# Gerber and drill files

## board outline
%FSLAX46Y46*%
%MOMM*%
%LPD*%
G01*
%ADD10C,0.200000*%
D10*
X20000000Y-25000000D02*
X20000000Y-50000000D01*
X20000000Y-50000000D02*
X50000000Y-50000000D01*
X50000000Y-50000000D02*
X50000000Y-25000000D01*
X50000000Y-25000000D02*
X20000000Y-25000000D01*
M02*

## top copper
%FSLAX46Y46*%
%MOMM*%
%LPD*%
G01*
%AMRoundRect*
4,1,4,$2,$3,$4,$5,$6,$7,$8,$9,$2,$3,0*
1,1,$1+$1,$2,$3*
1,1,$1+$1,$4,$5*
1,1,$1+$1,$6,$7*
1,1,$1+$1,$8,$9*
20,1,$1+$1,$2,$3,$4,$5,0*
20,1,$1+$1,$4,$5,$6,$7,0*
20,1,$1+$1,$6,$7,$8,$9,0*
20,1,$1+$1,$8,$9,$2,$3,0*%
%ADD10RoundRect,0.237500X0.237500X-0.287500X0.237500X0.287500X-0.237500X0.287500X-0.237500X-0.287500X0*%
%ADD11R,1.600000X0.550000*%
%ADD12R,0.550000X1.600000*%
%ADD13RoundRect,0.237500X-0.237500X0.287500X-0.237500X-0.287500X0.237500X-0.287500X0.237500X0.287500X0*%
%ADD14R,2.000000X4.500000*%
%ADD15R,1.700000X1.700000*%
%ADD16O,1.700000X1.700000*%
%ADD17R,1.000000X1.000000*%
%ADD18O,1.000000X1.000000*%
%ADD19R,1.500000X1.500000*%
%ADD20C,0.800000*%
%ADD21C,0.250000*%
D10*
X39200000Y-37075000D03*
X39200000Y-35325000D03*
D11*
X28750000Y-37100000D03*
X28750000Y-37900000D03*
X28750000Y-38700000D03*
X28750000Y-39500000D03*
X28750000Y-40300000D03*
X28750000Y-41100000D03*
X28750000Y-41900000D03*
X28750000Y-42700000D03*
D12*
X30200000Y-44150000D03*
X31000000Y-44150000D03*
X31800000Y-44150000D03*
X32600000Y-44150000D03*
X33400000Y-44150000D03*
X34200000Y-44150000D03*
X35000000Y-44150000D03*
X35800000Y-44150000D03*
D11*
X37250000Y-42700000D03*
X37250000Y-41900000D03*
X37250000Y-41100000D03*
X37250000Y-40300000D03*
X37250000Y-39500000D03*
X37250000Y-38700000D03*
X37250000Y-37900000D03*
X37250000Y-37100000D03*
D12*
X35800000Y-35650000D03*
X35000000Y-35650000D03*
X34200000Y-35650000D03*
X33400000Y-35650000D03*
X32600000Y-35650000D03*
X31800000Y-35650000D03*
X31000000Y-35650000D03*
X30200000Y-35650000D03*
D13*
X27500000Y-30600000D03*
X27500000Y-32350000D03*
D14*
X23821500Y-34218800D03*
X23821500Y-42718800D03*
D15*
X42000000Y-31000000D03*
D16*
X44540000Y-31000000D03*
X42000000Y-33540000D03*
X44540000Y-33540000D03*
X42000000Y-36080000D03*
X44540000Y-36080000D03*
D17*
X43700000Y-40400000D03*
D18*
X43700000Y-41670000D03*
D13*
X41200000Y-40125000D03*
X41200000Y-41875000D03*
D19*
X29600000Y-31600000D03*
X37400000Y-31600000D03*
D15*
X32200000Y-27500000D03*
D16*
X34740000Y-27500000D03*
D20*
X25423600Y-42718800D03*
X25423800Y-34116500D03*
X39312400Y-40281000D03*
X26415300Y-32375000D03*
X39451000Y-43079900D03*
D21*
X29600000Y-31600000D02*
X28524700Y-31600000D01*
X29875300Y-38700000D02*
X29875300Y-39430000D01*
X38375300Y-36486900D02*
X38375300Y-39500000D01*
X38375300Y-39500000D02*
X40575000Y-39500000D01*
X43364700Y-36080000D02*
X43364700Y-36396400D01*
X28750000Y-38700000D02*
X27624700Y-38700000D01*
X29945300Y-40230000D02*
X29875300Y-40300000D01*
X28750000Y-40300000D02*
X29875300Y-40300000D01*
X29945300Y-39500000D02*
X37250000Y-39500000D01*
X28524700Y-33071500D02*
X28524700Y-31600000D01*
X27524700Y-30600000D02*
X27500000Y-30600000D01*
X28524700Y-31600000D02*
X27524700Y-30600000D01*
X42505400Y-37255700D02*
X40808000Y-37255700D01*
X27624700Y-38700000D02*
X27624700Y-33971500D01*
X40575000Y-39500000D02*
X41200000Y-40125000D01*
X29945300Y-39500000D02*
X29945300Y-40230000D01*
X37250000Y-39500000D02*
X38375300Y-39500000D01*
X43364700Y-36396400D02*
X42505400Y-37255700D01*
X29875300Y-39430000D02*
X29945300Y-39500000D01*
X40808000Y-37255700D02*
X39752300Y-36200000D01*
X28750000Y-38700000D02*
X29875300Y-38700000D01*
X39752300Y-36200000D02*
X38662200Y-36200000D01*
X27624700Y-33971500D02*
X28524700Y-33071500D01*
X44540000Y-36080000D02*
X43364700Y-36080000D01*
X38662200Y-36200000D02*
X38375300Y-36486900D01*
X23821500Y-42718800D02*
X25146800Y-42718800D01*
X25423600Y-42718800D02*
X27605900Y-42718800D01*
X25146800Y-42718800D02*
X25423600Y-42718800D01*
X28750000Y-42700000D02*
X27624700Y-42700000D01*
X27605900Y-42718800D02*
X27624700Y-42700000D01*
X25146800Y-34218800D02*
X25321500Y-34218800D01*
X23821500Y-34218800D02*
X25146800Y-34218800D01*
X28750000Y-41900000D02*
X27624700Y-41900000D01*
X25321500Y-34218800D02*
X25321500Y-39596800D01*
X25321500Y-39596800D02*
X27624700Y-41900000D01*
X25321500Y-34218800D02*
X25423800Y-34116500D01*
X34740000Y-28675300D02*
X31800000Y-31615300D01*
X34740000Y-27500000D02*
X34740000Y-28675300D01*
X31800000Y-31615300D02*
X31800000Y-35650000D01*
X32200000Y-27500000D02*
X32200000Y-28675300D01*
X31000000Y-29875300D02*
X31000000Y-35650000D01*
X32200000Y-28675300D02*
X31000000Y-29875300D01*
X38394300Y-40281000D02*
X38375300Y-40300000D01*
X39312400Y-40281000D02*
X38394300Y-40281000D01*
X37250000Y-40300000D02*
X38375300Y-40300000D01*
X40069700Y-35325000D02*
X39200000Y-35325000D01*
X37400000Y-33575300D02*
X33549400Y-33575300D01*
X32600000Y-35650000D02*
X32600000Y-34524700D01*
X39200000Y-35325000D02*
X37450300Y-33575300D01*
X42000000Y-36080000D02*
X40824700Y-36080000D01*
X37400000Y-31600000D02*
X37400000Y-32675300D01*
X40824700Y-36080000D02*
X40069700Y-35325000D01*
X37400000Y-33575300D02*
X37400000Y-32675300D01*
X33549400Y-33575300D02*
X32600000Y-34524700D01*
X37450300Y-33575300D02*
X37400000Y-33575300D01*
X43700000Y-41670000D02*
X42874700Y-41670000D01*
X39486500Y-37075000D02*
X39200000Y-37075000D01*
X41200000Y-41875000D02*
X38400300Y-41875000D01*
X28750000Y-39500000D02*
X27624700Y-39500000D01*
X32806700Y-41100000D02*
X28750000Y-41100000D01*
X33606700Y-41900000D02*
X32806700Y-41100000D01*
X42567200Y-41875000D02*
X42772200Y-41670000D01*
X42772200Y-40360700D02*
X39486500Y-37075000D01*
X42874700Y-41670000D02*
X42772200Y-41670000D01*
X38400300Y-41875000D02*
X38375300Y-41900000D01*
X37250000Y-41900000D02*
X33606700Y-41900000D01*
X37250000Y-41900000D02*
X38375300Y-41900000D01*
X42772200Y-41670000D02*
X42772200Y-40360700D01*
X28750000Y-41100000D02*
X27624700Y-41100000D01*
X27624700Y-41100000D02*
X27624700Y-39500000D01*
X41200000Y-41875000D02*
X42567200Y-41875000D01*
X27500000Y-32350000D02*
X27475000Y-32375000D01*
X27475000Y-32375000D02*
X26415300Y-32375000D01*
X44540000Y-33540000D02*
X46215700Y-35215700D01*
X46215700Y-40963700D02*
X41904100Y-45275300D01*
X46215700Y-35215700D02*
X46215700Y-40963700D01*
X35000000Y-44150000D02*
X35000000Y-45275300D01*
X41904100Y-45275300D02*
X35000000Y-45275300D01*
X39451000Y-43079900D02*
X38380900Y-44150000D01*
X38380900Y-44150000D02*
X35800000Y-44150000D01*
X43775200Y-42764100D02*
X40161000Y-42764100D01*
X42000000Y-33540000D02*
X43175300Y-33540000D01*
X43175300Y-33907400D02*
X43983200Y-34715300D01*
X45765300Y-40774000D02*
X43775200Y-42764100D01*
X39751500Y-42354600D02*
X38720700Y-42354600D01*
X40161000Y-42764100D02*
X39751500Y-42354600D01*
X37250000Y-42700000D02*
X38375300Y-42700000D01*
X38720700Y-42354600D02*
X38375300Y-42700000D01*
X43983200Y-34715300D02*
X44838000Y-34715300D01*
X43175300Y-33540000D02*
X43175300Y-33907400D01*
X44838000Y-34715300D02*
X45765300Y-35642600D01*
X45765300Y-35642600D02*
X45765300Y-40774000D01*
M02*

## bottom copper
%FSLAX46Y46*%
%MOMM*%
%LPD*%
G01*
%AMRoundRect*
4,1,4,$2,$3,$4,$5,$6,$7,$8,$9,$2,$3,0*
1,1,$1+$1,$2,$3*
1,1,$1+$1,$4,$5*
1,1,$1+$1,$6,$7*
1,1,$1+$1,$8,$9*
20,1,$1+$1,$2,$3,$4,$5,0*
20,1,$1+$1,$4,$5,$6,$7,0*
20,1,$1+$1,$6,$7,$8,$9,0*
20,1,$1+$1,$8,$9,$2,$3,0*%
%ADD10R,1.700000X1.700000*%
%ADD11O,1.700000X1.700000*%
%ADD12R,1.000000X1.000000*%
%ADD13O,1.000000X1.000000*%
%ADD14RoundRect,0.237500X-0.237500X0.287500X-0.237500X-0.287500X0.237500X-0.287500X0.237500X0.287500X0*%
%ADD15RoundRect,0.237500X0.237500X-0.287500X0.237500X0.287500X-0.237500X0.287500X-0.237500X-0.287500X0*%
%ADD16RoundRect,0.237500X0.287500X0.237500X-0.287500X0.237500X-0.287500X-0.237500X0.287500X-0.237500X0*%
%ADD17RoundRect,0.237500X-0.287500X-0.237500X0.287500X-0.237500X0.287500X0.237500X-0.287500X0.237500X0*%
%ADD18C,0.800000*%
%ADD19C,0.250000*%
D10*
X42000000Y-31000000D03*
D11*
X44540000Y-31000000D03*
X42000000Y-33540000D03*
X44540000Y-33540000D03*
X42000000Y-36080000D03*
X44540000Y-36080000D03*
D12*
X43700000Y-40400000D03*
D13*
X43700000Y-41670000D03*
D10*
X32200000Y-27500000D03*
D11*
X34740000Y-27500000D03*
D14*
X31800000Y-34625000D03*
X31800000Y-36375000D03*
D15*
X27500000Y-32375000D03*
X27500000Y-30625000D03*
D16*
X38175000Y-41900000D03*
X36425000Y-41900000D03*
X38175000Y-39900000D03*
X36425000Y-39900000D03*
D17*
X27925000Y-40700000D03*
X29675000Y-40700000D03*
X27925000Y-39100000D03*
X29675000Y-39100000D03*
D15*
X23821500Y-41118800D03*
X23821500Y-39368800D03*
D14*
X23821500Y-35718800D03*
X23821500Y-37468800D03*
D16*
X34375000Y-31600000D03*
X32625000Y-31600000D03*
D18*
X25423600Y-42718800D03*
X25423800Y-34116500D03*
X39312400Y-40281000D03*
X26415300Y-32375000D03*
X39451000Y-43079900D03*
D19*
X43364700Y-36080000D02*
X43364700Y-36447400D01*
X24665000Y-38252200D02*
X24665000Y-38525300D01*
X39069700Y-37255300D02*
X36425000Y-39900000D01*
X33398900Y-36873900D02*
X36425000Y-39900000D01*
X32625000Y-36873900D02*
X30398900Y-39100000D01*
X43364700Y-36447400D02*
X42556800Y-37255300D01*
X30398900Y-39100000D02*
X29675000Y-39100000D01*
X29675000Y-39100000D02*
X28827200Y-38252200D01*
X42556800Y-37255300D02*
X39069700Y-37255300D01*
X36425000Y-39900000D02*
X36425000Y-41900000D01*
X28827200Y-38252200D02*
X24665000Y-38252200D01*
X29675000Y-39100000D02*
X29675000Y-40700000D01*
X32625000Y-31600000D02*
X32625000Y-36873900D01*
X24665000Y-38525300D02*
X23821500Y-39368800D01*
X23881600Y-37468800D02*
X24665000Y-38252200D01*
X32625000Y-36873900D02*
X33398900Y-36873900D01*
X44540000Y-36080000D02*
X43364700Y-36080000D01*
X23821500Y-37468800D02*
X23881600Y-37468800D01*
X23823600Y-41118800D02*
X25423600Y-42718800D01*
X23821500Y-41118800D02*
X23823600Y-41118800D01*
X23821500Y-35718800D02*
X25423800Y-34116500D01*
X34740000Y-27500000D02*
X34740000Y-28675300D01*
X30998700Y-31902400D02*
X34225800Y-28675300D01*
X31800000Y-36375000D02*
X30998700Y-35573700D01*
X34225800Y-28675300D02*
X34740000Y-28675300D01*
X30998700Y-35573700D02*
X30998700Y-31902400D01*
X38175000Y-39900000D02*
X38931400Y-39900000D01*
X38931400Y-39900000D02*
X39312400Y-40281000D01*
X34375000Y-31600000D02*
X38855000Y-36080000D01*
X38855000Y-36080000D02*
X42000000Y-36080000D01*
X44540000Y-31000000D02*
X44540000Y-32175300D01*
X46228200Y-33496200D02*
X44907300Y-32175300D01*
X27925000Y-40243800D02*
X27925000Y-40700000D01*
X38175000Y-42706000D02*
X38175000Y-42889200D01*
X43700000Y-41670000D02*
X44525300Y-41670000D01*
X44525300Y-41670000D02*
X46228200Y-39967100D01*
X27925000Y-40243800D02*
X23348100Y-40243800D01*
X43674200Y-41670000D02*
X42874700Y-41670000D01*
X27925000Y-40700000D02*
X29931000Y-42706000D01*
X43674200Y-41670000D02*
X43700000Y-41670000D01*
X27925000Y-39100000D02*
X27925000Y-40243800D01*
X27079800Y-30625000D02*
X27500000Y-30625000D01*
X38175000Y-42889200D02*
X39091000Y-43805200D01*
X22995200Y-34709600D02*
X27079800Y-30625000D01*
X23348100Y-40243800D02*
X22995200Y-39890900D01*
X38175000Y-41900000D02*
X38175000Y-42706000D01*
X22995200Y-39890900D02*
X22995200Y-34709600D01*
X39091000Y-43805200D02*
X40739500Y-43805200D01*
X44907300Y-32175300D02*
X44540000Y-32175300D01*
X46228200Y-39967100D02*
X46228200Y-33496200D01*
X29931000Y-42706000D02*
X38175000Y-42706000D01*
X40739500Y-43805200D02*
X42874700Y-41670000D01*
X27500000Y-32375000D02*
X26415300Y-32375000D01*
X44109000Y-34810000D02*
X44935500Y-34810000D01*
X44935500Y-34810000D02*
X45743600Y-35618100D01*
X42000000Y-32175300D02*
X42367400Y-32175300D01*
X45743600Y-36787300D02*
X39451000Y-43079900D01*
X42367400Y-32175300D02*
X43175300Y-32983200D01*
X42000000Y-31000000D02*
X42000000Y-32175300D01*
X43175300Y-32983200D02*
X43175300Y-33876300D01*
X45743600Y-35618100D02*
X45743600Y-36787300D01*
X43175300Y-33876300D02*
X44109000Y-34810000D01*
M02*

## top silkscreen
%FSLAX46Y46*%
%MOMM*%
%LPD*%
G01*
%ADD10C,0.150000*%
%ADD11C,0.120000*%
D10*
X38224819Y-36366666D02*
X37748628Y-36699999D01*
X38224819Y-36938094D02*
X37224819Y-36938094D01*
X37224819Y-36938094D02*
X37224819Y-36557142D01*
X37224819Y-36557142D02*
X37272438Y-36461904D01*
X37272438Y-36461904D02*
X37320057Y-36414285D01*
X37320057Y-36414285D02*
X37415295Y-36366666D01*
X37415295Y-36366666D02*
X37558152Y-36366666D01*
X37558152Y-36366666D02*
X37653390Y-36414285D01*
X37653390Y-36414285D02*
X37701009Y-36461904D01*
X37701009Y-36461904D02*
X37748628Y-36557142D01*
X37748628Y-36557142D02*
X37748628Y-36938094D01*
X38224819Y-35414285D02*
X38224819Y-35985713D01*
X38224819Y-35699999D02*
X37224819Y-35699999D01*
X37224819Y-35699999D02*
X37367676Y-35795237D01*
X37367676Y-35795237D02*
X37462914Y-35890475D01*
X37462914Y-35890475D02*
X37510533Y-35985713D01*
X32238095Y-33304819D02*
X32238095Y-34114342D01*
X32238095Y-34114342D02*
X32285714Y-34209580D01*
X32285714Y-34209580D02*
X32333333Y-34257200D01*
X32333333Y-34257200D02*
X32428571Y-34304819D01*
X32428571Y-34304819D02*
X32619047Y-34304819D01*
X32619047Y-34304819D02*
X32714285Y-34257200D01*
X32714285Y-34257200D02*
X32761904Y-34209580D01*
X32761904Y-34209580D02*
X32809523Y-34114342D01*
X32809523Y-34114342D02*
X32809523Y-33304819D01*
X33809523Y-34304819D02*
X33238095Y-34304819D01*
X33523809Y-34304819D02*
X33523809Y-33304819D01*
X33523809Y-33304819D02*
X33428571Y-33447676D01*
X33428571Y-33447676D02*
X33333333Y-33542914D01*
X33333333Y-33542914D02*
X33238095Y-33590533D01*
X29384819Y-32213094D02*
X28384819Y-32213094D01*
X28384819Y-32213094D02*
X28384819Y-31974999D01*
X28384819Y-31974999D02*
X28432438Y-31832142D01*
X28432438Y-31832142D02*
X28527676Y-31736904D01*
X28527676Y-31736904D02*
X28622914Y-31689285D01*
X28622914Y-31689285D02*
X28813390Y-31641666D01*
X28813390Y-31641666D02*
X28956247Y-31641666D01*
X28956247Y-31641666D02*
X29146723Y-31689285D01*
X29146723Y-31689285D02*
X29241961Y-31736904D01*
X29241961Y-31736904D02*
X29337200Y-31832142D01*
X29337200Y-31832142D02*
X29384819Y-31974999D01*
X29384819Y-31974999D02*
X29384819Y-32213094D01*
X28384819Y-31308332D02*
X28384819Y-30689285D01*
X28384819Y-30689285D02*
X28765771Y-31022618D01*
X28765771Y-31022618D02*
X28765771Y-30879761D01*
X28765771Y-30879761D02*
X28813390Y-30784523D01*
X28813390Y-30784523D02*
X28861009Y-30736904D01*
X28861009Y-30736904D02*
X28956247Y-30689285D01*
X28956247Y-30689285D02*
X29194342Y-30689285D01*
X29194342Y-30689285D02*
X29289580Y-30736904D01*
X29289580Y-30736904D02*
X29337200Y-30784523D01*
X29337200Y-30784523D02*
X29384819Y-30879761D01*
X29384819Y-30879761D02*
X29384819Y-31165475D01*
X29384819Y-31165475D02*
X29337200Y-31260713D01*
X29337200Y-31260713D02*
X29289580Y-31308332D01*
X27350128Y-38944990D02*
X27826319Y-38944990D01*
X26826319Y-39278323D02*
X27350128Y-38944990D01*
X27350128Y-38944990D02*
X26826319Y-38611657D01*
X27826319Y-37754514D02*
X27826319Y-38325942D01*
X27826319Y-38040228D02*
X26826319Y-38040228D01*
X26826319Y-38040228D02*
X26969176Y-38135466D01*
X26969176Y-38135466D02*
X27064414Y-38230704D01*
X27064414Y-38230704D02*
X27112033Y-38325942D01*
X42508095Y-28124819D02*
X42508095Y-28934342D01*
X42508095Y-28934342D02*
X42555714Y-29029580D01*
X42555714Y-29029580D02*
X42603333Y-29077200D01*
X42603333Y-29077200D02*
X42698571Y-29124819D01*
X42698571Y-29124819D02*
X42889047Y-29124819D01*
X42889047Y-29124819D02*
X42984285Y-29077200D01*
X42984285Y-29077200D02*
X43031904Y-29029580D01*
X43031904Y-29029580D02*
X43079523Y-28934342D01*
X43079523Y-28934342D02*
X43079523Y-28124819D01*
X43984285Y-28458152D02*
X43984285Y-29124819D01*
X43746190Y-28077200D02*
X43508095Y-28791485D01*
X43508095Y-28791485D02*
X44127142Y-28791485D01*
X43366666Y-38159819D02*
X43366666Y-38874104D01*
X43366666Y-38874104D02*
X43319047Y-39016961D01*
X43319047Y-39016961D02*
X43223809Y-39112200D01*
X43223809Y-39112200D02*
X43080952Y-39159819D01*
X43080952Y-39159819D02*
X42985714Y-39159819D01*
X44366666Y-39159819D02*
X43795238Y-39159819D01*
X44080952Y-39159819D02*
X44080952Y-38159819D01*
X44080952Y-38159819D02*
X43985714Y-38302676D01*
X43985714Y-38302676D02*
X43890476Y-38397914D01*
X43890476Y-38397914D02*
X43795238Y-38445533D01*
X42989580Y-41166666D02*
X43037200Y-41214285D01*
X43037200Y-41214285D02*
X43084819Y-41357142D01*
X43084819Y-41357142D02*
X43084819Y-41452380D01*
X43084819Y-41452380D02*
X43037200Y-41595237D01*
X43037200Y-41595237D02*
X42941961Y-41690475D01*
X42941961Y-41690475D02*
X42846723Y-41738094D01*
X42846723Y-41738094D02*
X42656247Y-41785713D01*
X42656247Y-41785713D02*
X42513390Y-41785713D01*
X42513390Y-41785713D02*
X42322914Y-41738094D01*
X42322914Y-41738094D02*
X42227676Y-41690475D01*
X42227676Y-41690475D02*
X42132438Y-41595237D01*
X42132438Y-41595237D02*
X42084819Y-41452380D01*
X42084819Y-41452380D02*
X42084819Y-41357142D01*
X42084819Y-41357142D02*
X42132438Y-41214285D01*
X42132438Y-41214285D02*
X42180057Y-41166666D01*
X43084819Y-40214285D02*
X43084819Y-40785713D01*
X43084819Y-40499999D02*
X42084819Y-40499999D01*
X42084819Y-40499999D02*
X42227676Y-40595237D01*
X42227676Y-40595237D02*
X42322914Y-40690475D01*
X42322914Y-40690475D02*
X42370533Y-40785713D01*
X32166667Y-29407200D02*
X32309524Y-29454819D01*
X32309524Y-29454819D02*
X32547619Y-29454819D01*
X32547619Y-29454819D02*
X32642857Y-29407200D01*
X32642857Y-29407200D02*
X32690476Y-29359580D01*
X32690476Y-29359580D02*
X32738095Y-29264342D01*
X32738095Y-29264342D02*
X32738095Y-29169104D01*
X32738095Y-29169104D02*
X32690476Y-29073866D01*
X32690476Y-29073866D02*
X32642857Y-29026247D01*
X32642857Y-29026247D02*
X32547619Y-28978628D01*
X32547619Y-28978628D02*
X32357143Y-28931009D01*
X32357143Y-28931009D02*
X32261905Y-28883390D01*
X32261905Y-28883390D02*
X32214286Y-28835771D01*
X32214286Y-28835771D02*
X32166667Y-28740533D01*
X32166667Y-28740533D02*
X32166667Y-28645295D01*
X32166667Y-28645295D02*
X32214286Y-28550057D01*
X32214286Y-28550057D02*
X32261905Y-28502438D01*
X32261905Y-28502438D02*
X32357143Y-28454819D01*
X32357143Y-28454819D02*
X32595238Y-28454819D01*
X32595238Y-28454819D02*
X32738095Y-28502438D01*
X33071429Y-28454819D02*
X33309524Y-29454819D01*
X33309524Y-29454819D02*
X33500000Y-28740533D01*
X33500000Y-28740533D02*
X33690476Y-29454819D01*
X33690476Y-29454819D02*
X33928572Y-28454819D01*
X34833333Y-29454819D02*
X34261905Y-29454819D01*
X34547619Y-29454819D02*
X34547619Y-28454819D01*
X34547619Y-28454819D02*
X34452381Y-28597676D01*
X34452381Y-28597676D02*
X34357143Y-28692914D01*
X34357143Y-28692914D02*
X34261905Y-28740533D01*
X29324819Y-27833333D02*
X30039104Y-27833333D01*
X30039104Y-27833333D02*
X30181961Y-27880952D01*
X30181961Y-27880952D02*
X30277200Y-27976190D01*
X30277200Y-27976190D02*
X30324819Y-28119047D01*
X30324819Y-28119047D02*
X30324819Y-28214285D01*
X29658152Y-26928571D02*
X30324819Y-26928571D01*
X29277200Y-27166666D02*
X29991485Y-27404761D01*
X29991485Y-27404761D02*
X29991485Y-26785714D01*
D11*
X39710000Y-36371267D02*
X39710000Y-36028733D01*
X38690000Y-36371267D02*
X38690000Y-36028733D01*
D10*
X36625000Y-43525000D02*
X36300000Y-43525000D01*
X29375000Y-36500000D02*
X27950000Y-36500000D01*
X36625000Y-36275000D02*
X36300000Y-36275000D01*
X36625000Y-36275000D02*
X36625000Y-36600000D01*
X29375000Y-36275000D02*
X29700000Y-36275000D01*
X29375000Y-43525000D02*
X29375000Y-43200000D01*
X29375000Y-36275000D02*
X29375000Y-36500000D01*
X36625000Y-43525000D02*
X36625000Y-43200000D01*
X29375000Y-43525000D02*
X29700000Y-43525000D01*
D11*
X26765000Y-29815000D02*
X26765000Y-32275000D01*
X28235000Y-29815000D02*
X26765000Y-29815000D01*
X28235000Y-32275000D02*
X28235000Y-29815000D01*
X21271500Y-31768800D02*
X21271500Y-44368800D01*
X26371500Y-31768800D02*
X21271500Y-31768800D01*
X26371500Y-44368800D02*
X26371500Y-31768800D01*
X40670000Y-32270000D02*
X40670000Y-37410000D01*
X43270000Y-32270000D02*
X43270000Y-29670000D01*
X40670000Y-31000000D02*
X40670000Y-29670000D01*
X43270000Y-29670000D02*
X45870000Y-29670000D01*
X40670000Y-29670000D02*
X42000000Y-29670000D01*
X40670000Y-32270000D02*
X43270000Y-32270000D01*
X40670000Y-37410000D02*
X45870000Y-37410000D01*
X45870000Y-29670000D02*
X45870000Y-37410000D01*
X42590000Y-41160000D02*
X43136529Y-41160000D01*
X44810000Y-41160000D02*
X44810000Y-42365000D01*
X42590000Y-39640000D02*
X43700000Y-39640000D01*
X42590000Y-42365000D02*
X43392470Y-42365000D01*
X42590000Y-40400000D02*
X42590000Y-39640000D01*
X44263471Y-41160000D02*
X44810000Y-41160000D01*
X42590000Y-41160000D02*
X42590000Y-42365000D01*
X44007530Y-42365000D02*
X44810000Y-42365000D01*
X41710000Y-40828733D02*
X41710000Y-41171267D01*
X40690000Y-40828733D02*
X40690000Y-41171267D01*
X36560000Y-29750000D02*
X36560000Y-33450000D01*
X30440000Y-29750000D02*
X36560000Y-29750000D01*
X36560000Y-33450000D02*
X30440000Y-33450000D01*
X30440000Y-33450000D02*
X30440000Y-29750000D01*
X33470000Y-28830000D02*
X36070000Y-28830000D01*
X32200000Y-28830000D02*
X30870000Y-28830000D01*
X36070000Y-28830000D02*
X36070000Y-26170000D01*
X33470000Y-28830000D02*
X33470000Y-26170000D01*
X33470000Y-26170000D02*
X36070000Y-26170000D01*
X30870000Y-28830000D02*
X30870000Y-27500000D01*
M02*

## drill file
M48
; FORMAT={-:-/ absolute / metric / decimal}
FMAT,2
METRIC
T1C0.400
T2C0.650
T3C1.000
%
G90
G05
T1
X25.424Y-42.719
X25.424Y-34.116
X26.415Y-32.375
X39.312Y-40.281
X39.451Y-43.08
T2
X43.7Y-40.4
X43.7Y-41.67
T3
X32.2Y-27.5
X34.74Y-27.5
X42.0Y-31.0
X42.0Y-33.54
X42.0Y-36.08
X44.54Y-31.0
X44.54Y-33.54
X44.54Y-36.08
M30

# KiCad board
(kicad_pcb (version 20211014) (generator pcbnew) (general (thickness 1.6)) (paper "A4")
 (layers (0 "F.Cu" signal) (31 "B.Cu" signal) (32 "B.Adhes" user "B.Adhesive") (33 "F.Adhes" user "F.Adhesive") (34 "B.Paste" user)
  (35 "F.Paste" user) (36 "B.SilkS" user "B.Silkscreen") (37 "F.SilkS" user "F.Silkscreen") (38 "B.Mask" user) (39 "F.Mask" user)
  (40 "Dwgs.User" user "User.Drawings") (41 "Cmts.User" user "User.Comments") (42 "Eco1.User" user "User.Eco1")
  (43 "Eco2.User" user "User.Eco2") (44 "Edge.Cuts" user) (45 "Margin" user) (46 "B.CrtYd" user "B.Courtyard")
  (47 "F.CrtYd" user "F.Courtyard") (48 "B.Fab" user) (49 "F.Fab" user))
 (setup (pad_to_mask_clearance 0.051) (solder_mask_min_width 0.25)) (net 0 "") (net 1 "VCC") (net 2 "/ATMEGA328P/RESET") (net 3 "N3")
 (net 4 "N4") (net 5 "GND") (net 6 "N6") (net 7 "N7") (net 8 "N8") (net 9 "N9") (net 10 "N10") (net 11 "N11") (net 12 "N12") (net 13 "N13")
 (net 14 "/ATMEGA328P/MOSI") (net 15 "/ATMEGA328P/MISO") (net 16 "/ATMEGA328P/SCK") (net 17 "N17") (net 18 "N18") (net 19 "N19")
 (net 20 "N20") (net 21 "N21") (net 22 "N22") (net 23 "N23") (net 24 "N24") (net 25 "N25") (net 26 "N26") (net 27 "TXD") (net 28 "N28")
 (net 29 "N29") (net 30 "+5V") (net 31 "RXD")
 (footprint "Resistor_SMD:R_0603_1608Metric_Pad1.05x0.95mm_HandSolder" (layer "F.Cu") (at 39.2 36.2 90)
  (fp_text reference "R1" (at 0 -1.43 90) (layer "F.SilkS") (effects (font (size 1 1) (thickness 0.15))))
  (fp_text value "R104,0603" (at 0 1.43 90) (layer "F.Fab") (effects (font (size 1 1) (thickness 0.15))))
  (fp_line (start -0.171267 0.51) (end 0.171267 0.51) (layer "F.SilkS") (width 0.12))
  (fp_line (start -0.171267 -0.51) (end 0.171267 -0.51) (layer "F.SilkS") (width 0.12))
  (pad "1" smd roundrect locked (at -0.875 0 90) (size 1.05 0.95) (layers "F.Cu" "F.Paste" "F.Mask") (roundrect_rratio 0.25) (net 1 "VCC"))
  (pad "2" smd roundrect locked (at 0.875 0 90) (size 1.05 0.95) (layers "F.Cu" "F.Paste" "F.Mask") (roundrect_rratio 0.25)
   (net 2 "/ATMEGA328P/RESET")))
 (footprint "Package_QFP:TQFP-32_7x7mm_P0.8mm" (layer "F.Cu") (at 33 39.9)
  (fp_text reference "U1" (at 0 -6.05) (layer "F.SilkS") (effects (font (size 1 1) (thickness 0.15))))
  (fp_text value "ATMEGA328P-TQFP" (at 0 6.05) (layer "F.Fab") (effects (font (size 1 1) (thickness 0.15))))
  (fp_line (start 3.625 3.625) (end 3.3 3.625) (layer "F.SilkS") (width 0.15))
  (fp_line (start -3.625 -3.4) (end -5.05 -3.4) (layer "F.SilkS") (width 0.15))
  (fp_line (start 3.625 -3.625) (end 3.3 -3.625) (layer "F.SilkS") (width 0.15))
  (fp_line (start 3.625 -3.625) (end 3.625 -3.3) (layer "F.SilkS") (width 0.15))
  (fp_line (start -3.625 -3.625) (end -3.3 -3.625) (layer "F.SilkS") (width 0.15))
  (fp_line (start -3.625 3.625) (end -3.625 3.3) (layer "F.SilkS") (width 0.15))
  (fp_line (start -3.625 -3.625) (end -3.625 -3.4) (layer "F.SilkS") (width 0.15))
  (fp_line (start 3.625 3.625) (end 3.625 3.3) (layer "F.SilkS") (width 0.15))
  (fp_line (start -3.625 3.625) (end -3.3 3.625) (layer "F.SilkS") (width 0.15))
  (pad "1" smd rect locked (at -4.25 -2.8) (size 1.6 0.55) (layers "F.Cu" "F.Paste" "F.Mask") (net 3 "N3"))
  (pad "2" smd rect locked (at -4.25 -2) (size 1.6 0.55) (layers "F.Cu" "F.Paste" "F.Mask") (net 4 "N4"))
  (pad "3" smd rect locked (at -4.25 -1.2) (size 1.6 0.55) (layers "F.Cu" "F.Paste" "F.Mask") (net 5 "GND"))
  (pad "4" smd rect locked (at -4.25 -0.4) (size 1.6 0.55) (layers "F.Cu" "F.Paste" "F.Mask") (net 1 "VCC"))
  (pad "5" smd rect locked (at -4.25 0.4) (size 1.6 0.55) (layers "F.Cu" "F.Paste" "F.Mask") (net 5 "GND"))
  (pad "6" smd rect locked (at -4.25 1.2) (size 1.6 0.55) (layers "F.Cu" "F.Paste" "F.Mask") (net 1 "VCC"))
  (pad "7" smd rect locked (at -4.25 2) (size 1.6 0.55) (layers "F.Cu" "F.Paste" "F.Mask") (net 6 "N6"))
  (pad "8" smd rect locked (at -4.25 2.8) (size 1.6 0.55) (layers "F.Cu" "F.Paste" "F.Mask") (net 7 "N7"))
  (pad "9" smd rect locked (at -2.8 4.25 90) (size 1.6 0.55) (layers "F.Cu" "F.Paste" "F.Mask") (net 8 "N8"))
  (pad "10" smd rect locked (at -2 4.25 90) (size 1.6 0.55) (layers "F.Cu" "F.Paste" "F.Mask") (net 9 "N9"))
  (pad "11" smd rect locked (at -1.2 4.25 90) (size 1.6 0.55) (layers "F.Cu" "F.Paste" "F.Mask") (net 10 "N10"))
  (pad "12" smd rect locked (at -0.4 4.25 90) (size 1.6 0.55) (layers "F.Cu" "F.Paste" "F.Mask") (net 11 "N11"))
  (pad "13" smd rect locked (at 0.4 4.25 90) (size 1.6 0.55) (layers "F.Cu" "F.Paste" "F.Mask") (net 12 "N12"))
  (pad "14" smd rect locked (at 1.2 4.25 90) (size 1.6 0.55) (layers "F.Cu" "F.Paste" "F.Mask") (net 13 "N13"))
  (pad "15" smd rect locked (at 2 4.25 90) (size 1.6 0.55) (layers "F.Cu" "F.Paste" "F.Mask") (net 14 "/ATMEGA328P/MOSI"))
  (pad "16" smd rect locked (at 2.8 4.25 90) (size 1.6 0.55) (layers "F.Cu" "F.Paste" "F.Mask") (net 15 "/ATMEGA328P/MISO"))
  (pad "17" smd rect locked (at 4.25 2.8) (size 1.6 0.55) (layers "F.Cu" "F.Paste" "F.Mask") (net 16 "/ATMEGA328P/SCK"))
  (pad "18" smd rect locked (at 4.25 2) (size 1.6 0.55) (layers "F.Cu" "F.Paste" "F.Mask") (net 1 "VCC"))
  (pad "19" smd rect locked (at 4.25 1.2) (size 1.6 0.55) (layers "F.Cu" "F.Paste" "F.Mask") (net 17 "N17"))
  (pad "20" smd rect locked (at 4.25 0.4) (size 1.6 0.55) (layers "F.Cu" "F.Paste" "F.Mask") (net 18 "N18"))
  (pad "21" smd rect locked (at 4.25 -0.4) (size 1.6 0.55) (layers "F.Cu" "F.Paste" "F.Mask") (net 5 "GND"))
  (pad "22" smd rect locked (at 4.25 -1.2) (size 1.6 0.55) (layers "F.Cu" "F.Paste" "F.Mask") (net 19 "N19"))
  (pad "23" smd rect locked (at 4.25 -2) (size 1.6 0.55) (layers "F.Cu" "F.Paste" "F.Mask") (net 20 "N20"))
  (pad "24" smd rect locked (at 4.25 -2.8) (size 1.6 0.55) (layers "F.Cu" "F.Paste" "F.Mask") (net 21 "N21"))
  (pad "25" smd rect locked (at 2.8 -4.25 90) (size 1.6 0.55) (layers "F.Cu" "F.Paste" "F.Mask") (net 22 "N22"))
  (pad "26" smd rect locked (at 2 -4.25 90) (size 1.6 0.55) (layers "F.Cu" "F.Paste" "F.Mask") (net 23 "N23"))
  (pad "27" smd rect locked (at 1.2 -4.25 90) (size 1.6 0.55) (layers "F.Cu" "F.Paste" "F.Mask") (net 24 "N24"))
  (pad "28" smd rect locked (at 0.4 -4.25 90) (size 1.6 0.55) (layers "F.Cu" "F.Paste" "F.Mask") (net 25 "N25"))
  (pad "29" smd rect locked (at -0.4 -4.25 90) (size 1.6 0.55) (layers "F.Cu" "F.Paste" "F.Mask") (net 2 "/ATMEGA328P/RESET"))
  (pad "30" smd rect locked (at -1.2 -4.25 90) (size 1.6 0.55) (layers "F.Cu" "F.Paste" "F.Mask") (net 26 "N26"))
  (pad "31" smd rect locked (at -2 -4.25 90) (size 1.6 0.55) (layers "F.Cu" "F.Paste" "F.Mask") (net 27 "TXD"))
  (pad "32" smd rect locked (at -2.8 -4.25 90) (size 1.6 0.55) (layers "F.Cu" "F.Paste" "F.Mask") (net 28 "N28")))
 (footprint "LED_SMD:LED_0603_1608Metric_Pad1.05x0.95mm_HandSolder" (layer "F.Cu") (at 27.5 31.475 -90)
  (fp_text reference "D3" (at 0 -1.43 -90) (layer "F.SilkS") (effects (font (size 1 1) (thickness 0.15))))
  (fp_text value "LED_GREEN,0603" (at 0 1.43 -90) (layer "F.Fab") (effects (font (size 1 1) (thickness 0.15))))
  (fp_line (start -1.66 0.735) (end 0.8 0.735) (layer "F.SilkS") (width 0.12))
  (fp_line (start -1.66 -0.735) (end -1.66 0.735) (layer "F.SilkS") (width 0.12))
  (fp_line (start 0.8 -0.735) (end -1.66 -0.735) (layer "F.SilkS") (width 0.12))
  (pad "1" smd roundrect locked (at -0.875 0 270) (size 1.05 0.95) (layers "F.Cu" "F.Paste" "F.Mask") (roundrect_rratio 0.25) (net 5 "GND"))
  (pad "2" smd roundrect locked (at 0.875 0 270) (size 1.05 0.95) (layers "F.Cu" "F.Paste" "F.Mask") (roundrect_rratio 0.25) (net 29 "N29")))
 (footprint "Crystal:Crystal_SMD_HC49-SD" (layer "F.Cu") (at 23.8215 38.4688 -90)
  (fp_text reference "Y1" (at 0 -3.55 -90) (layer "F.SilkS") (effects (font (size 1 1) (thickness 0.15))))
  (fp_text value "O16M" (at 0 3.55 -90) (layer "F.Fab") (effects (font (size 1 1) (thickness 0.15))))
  (fp_line (start -6.7 2.55) (end 5.9 2.55) (layer "F.SilkS") (width 0.12))
  (fp_line (start -6.7 -2.55) (end -6.7 2.55) (layer "F.SilkS") (width 0.12))
  (fp_line (start 5.9 -2.55) (end -6.7 -2.55) (layer "F.SilkS") (width 0.12))
  (pad "1" smd rect locked (at -4.25 0 270) (size 4.5 2) (layers "F.Cu" "F.Paste" "F.Mask") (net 6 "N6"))
  (pad "2" smd rect locked (at 4.25 0 270) (size 4.5 2) (layers "F.Cu" "F.Paste" "F.Mask") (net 7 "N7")))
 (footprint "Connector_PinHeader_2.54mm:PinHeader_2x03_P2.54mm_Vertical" (layer "F.Cu") (at 42 31)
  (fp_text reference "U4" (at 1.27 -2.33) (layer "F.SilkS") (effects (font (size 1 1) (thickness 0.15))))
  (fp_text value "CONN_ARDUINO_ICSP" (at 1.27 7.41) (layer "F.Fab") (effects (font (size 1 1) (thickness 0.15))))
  (fp_line (start -1.33 1.27) (end -1.33 6.41) (layer "F.SilkS") (width 0.12))
  (fp_line (start 1.27 1.27) (end 1.27 -1.33) (layer "F.SilkS") (width 0.12))
  (fp_line (start -1.33 0) (end -1.33 -1.33) (layer "F.SilkS") (width 0.12))
  (fp_line (start 1.27 -1.33) (end 3.87 -1.33) (layer "F.SilkS") (width 0.12))
  (fp_line (start -1.33 -1.33) (end 0 -1.33) (layer "F.SilkS") (width 0.12))
  (fp_line (start -1.33 1.27) (end 1.27 1.27) (layer "F.SilkS") (width 0.12))
  (fp_line (start -1.33 6.41) (end 3.87 6.41) (layer "F.SilkS") (width 0.12))
  (fp_line (start 3.87 -1.33) (end 3.87 6.41) (layer "F.SilkS") (width 0.12))
  (pad "1" thru_hole rect locked (at 0 0) (size 1.7 1.7) (drill 1) (layers *.Cu *.Mask) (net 15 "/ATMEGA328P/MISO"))
  (pad "2" thru_hole oval locked (at 2.54 0) (size 1.7 1.7) (drill 1) (layers *.Cu *.Mask) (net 1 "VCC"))
  (pad "3" thru_hole oval locked (at 0 2.54) (size 1.7 1.7) (drill 1) (layers *.Cu *.Mask) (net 16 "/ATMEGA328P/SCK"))
  (pad "4" thru_hole oval locked (at 2.54 2.54) (size 1.7 1.7) (drill 1) (layers *.Cu *.Mask) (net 14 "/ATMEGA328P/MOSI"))
  (pad "5" thru_hole oval locked (at 0 5.08) (size 1.7 1.7) (drill 1) (layers *.Cu *.Mask) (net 2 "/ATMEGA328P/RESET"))
  (pad "6" thru_hole oval locked (at 2.54 5.08) (size 1.7 1.7) (drill 1) (layers *.Cu *.Mask) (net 5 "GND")))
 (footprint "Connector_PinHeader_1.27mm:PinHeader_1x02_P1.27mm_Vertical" (layer "F.Cu") (at 43.7 40.4)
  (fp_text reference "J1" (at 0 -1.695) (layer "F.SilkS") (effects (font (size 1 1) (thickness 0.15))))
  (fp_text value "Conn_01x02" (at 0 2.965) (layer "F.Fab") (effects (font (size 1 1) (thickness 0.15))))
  (fp_line (start -1.11 0.76) (end -0.563471 0.76) (layer "F.SilkS") (width 0.12))
  (fp_line (start 1.11 0.76) (end 1.11 1.965) (layer "F.SilkS") (width 0.12))
  (fp_line (start -1.11 -0.76) (end 0 -0.76) (layer "F.SilkS") (width 0.12))
  (fp_line (start -1.11 1.965) (end -0.30753 1.965) (layer "F.SilkS") (width 0.12))
  (fp_line (start -1.11 0) (end -1.11 -0.76) (layer "F.SilkS") (width 0.12))
  (fp_line (start 0.563471 0.76) (end 1.11 0.76) (layer "F.SilkS") (width 0.12))
  (fp_line (start -1.11 0.76) (end -1.11 1.965) (layer "F.SilkS") (width 0.12))
  (fp_line (start 0.30753 1.965) (end 1.11 1.965) (layer "F.SilkS") (width 0.12))
  (pad "1" thru_hole rect locked (at 0 0) (size 1 1) (drill 0.65) (layers *.Cu *.Mask) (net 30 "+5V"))
  (pad "2" thru_hole oval locked (at 0 1.27) (size 1 1) (drill 0.65) (layers *.Cu *.Mask) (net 1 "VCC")))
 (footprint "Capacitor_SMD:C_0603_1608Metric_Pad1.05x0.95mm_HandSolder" (layer "F.Cu") (at 41.2 41 -90)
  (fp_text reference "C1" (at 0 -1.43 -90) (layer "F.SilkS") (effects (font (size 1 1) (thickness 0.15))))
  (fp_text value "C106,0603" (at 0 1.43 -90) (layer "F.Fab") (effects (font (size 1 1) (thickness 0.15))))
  (fp_line (start -0.171267 -0.51) (end 0.171267 -0.51) (layer "F.SilkS") (width 0.12))
  (fp_line (start -0.171267 0.51) (end 0.171267 0.51) (layer "F.SilkS") (width 0.12))
  (pad "1" smd roundrect locked (at -0.875 0 270) (size 1.05 0.95) (layers "F.Cu" "F.Paste" "F.Mask") (roundrect_rratio 0.25) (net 5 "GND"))
  (pad "2" smd roundrect locked (at 0.875 0 270) (size 1.05 0.95) (layers "F.Cu" "F.Paste" "F.Mask") (roundrect_rratio 0.25) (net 1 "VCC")))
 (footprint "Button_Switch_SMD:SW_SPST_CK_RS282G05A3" (layer "F.Cu") (at 33.5 31.6)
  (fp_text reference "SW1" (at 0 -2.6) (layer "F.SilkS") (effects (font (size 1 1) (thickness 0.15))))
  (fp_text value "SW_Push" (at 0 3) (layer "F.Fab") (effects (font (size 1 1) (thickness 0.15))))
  (fp_line (start 3.06 -1.85) (end 3.06 1.85) (layer "F.SilkS") (width 0.12))
  (fp_line (start -3.06 -1.85) (end 3.06 -1.85) (layer "F.SilkS") (width 0.12))
  (fp_line (start 3.06 1.85) (end -3.06 1.85) (layer "F.SilkS") (width 0.12))
  (fp_line (start -3.06 1.85) (end -3.06 -1.85) (layer "F.SilkS") (width 0.12))
  (pad "1" smd rect locked (at -3.9 0) (size 1.5 1.5) (layers "F.Cu" "F.Paste" "F.Mask") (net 5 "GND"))
  (pad "2" smd rect locked (at 3.9 0) (size 1.5 1.5) (layers "F.Cu" "F.Paste" "F.Mask") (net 2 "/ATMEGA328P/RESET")))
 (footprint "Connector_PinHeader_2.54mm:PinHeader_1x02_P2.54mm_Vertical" (layer "F.Cu") (at 32.2 27.5 90)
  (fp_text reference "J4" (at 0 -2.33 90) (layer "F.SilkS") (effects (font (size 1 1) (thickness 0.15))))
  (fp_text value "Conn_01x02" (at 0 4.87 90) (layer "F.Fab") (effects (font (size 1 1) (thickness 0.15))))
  (fp_line (start -1.33 1.27) (end -1.33 3.87) (layer "F.SilkS") (width 0.12))
  (fp_line (start -1.33 0) (end -1.33 -1.33) (layer "F.SilkS") (width 0.12))
  (fp_line (start -1.33 3.87) (end 1.33 3.87) (layer "F.SilkS") (width 0.12))
  (fp_line (start -1.33 1.27) (end 1.33 1.27) (layer "F.SilkS") (width 0.12))
  (fp_line (start 1.33 1.27) (end 1.33 3.87) (layer "F.SilkS") (width 0.12))
  (fp_line (start -1.33 -1.33) (end 0 -1.33) (layer "F.SilkS") (width 0.12))
  (pad "1" thru_hole rect locked (at 0 0 90) (size 1.7 1.7) (drill 1) (layers *.Cu *.Mask) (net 27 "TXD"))
  (pad "2" thru_hole oval locked (at 0 2.54 90) (size 1.7 1.7) (drill 1) (layers *.Cu *.Mask) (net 26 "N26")))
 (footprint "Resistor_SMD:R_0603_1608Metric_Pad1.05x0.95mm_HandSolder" (layer "B.Cu") (at 31.8 35.5 -90)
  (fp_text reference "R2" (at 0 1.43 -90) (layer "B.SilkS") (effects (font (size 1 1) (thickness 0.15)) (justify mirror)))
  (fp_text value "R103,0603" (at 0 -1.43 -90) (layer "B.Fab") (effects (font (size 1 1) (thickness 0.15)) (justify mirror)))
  (pad "1" smd roundrect locked (at -0.875 0 270) (size 1.05 0.95) (layers "B.Cu" "B.Paste" "B.Mask") (roundrect_rratio 0.25) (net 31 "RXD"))
  (pad "2" smd roundrect locked (at 0.875 0 270) (size 1.05 0.95) (layers "B.Cu" "B.Paste" "B.Mask") (roundrect_rratio 0.25) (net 26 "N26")))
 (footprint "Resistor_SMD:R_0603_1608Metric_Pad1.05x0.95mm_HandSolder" (layer "B.Cu") (at 27.5 31.5 90)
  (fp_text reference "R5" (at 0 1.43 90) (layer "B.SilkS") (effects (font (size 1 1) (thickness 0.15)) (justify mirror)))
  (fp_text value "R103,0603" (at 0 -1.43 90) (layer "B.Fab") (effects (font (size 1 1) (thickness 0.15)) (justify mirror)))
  (pad "1" smd roundrect locked (at -0.875 0 90) (size 1.05 0.95) (layers "B.Cu" "B.Paste" "B.Mask") (roundrect_rratio 0.25) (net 29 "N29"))
  (pad "2" smd roundrect locked (at 0.875 0 90) (size 1.05 0.95) (layers "B.Cu" "B.Paste" "B.Mask") (roundrect_rratio 0.25) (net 1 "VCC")))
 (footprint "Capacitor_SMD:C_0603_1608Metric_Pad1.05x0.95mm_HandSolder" (layer "B.Cu") (at 37.3 41.9 180)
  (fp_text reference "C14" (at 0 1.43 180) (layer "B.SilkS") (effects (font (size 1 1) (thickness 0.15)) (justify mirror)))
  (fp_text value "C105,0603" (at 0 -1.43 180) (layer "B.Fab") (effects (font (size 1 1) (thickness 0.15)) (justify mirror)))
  (pad "1" smd roundrect locked (at -0.875 0 180) (size 1.05 0.95) (layers "B.Cu" "B.Paste" "B.Mask") (roundrect_rratio 0.25) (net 1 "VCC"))
  (pad "2" smd roundrect locked (at 0.875 0 180) (size 1.05 0.95) (layers "B.Cu" "B.Paste" "B.Mask") (roundrect_rratio 0.25) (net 5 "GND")))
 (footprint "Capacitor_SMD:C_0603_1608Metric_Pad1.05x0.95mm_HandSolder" (layer "B.Cu") (at 37.3 39.9 180)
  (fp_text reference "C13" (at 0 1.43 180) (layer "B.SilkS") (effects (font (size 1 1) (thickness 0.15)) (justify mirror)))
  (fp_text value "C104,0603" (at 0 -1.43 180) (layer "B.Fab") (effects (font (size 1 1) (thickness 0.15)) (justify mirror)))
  (pad "1" smd roundrect locked (at -0.875 0 180) (size 1.05 0.95) (layers "B.Cu" "B.Paste" "B.Mask") (roundrect_rratio 0.25) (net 18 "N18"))
  (pad "2" smd roundrect locked (at 0.875 0 180) (size 1.05 0.95) (layers "B.Cu" "B.Paste" "B.Mask") (roundrect_rratio 0.25) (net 5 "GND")))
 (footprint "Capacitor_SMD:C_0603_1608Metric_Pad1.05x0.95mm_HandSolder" (layer "B.Cu") (at 28.8 40.7)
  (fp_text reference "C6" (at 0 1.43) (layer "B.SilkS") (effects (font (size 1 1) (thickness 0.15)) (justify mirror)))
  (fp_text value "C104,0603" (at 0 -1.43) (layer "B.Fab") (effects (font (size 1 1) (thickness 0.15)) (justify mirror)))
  (pad "1" smd roundrect locked (at -0.875 0) (size 1.05 0.95) (layers "B.Cu" "B.Paste" "B.Mask") (roundrect_rratio 0.25) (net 1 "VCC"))
  (pad "2" smd roundrect locked (at 0.875 0) (size 1.05 0.95) (layers "B.Cu" "B.Paste" "B.Mask") (roundrect_rratio 0.25) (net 5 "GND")))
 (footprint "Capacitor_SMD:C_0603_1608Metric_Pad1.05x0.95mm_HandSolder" (layer "B.Cu") (at 28.8 39.1)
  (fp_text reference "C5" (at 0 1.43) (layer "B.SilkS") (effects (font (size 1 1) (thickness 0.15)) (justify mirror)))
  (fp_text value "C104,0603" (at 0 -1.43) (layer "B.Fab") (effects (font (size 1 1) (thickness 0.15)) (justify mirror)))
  (pad "1" smd roundrect locked (at -0.875 0) (size 1.05 0.95) (layers "B.Cu" "B.Paste" "B.Mask") (roundrect_rratio 0.25) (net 1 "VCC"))
  (pad "2" smd roundrect locked (at 0.875 0) (size 1.05 0.95) (layers "B.Cu" "B.Paste" "B.Mask") (roundrect_rratio 0.25) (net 5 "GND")))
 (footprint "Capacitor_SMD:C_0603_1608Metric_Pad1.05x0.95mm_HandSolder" (layer "B.Cu") (at 23.8215 40.2438 90)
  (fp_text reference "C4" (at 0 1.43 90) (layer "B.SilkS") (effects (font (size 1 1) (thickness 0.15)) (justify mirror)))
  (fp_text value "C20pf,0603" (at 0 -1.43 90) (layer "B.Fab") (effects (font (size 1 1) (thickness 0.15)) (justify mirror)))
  (pad "1" smd roundrect locked (at -0.875 0 90) (size 1.05 0.95) (layers "B.Cu" "B.Paste" "B.Mask") (roundrect_rratio 0.25) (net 7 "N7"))
  (pad "2" smd roundrect locked (at 0.875 0 90) (size 1.05 0.95) (layers "B.Cu" "B.Paste" "B.Mask") (roundrect_rratio 0.25) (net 5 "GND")))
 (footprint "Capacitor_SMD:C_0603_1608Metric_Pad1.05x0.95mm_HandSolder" (layer "B.Cu") (at 23.8215 36.5938 -90)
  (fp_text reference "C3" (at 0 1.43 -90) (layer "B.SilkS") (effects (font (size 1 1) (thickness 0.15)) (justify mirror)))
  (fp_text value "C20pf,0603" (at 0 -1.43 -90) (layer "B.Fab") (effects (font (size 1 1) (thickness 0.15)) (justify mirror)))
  (pad "1" smd roundrect locked (at -0.875 0 270) (size 1.05 0.95) (layers "B.Cu" "B.Paste" "B.Mask") (roundrect_rratio 0.25) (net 6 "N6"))
  (pad "2" smd roundrect locked (at 0.875 0 270) (size 1.05 0.95) (layers "B.Cu" "B.Paste" "B.Mask") (roundrect_rratio 0.25) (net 5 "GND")))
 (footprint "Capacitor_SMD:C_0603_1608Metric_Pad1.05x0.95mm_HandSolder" (layer "B.Cu") (at 33.5 31.6 180)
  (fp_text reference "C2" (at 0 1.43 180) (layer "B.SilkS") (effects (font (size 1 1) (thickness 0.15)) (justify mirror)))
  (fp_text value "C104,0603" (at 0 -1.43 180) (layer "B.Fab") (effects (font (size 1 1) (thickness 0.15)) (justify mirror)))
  (pad "1" smd roundrect locked (at -0.875 0 180) (size 1.05 0.95) (layers "B.Cu" "B.Paste" "B.Mask") (roundrect_rratio 0.25)
   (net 2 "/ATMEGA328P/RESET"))
  (pad "2" smd roundrect locked (at 0.875 0 180) (size 1.05 0.95) (layers "B.Cu" "B.Paste" "B.Mask") (roundrect_rratio 0.25) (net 5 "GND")))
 (gr_line (start 20 25) (end 20 50) (layer "Edge.Cuts") (width 0.2))
 (gr_line (start 20 50) (end 50 50) (layer "Edge.Cuts") (width 0.2))
 (gr_line (start 50 50) (end 50 25) (layer "Edge.Cuts") (width 0.2))
 (gr_line (start 50 25) (end 20 25) (layer "Edge.Cuts") (width 0.2))
 (segment (start 29.6 31.6) (end 28.5247 31.6) (width 0.25) (layer "F.Cu") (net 5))
 (segment (start 29.8753 38.7) (end 29.8753 39.43) (width 0.25) (layer "F.Cu") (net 5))
 (segment (start 38.3753 36.4869) (end 38.3753 39.5) (width 0.25) (layer "F.Cu") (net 5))
 (segment (start 38.3753 39.5) (end 40.575 39.5) (width 0.25) (layer "F.Cu") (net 5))
 (segment (start 43.3647 36.08) (end 43.3647 36.3964) (width 0.25) (layer "F.Cu") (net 5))
 (segment (start 28.75 38.7) (end 27.6247 38.7) (width 0.25) (layer "F.Cu") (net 5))
 (segment (start 29.9453 40.23) (end 29.8753 40.3) (width 0.25) (layer "F.Cu") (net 5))
 (segment (start 28.75 40.3) (end 29.8753 40.3) (width 0.25) (layer "F.Cu") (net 5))
 (segment (start 29.9453 39.5) (end 37.25 39.5) (width 0.25) (layer "F.Cu") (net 5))
 (segment (start 28.5247 33.0715) (end 28.5247 31.6) (width 0.25) (layer "F.Cu") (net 5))
 (segment (start 27.5247 30.6) (end 27.5 30.6) (width 0.25) (layer "F.Cu") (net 5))
 (segment (start 28.5247 31.6) (end 27.5247 30.6) (width 0.25) (layer "F.Cu") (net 5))
 (segment (start 42.5054 37.2557) (end 40.808 37.2557) (width 0.25) (layer "F.Cu") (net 5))
 (segment (start 27.6247 38.7) (end 27.6247 33.9715) (width 0.25) (layer "F.Cu") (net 5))
 (segment (start 40.575 39.5) (end 41.2 40.125) (width 0.25) (layer "F.Cu") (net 5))
 (segment (start 29.9453 39.5) (end 29.9453 40.23) (width 0.25) (layer "F.Cu") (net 5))
 (segment (start 37.25 39.5) (end 38.3753 39.5) (width 0.25) (layer "F.Cu") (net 5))
 (segment (start 43.3647 36.3964) (end 42.5054 37.2557) (width 0.25) (layer "F.Cu") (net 5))
 (segment (start 29.8753 39.43) (end 29.9453 39.5) (width 0.25) (layer "F.Cu") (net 5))
 (segment (start 40.808 37.2557) (end 39.7523 36.2) (width 0.25) (layer "F.Cu") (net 5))
 (segment (start 28.75 38.7) (end 29.8753 38.7) (width 0.25) (layer "F.Cu") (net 5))
 (segment (start 39.7523 36.2) (end 38.6622 36.2) (width 0.25) (layer "F.Cu") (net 5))
 (segment (start 27.6247 33.9715) (end 28.5247 33.0715) (width 0.25) (layer "F.Cu") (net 5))
 (segment (start 44.54 36.08) (end 43.3647 36.08) (width 0.25) (layer "F.Cu") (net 5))
 (segment (start 38.6622 36.2) (end 38.3753 36.4869) (width 0.25) (layer "F.Cu") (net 5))
 (segment (start 43.3647 36.08) (end 43.3647 36.4474) (width 0.25) (layer "B.Cu") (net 5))
 (segment (start 24.665 38.2522) (end 24.665 38.5253) (width 0.25) (layer "B.Cu") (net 5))
 (segment (start 39.0697 37.2553) (end 36.425 39.9) (width 0.25) (layer "B.Cu") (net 5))
 (segment (start 33.3989 36.8739) (end 36.425 39.9) (width 0.25) (layer "B.Cu") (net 5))
 (segment (start 32.625 36.8739) (end 30.3989 39.1) (width 0.25) (layer "B.Cu") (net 5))
 (segment (start 43.3647 36.4474) (end 42.5568 37.2553) (width 0.25) (layer "B.Cu") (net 5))
 (segment (start 30.3989 39.1) (end 29.675 39.1) (width 0.25) (layer "B.Cu") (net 5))
 (segment (start 29.675 39.1) (end 28.8272 38.2522) (width 0.25) (layer "B.Cu") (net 5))
 (segment (start 42.5568 37.2553) (end 39.0697 37.2553) (width 0.25) (layer "B.Cu") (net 5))
 (segment (start 36.425 39.9) (end 36.425 41.9) (width 0.25) (layer "B.Cu") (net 5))
 (segment (start 28.8272 38.2522) (end 24.665 38.2522) (width 0.25) (layer "B.Cu") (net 5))
 (segment (start 29.675 39.1) (end 29.675 40.7) (width 0.25) (layer "B.Cu") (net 5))
 (segment (start 32.625 31.6) (end 32.625 36.8739) (width 0.25) (layer "B.Cu") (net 5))
 (segment (start 24.665 38.5253) (end 23.8215 39.3688) (width 0.25) (layer "B.Cu") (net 5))
 (segment (start 23.8816 37.4688) (end 24.665 38.2522) (width 0.25) (layer "B.Cu") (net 5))
 (segment (start 32.625 36.8739) (end 33.3989 36.8739) (width 0.25) (layer "B.Cu") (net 5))
 (segment (start 44.54 36.08) (end 43.3647 36.08) (width 0.25) (layer "B.Cu") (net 5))
 (segment (start 23.8215 37.4688) (end 23.8816 37.4688) (width 0.25) (layer "B.Cu") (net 5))
 (segment (start 23.8215 42.7188) (end 25.1468 42.7188) (width 0.25) (layer "F.Cu") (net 7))
 (segment (start 25.4236 42.7188) (end 27.6059 42.7188) (width 0.25) (layer "F.Cu") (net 7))
 (segment (start 25.1468 42.7188) (end 25.4236 42.7188) (width 0.25) (layer "F.Cu") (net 7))
 (segment (start 28.75 42.7) (end 27.6247 42.7) (width 0.25) (layer "F.Cu") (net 7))
 (segment (start 27.6059 42.7188) (end 27.6247 42.7) (width 0.25) (layer "F.Cu") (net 7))
 (via (at 25.4236 42.7188) (size 0.8) (drill 0.4) (layers "F.Cu" "B.Cu") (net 7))
 (segment (start 23.8236 41.1188) (end 25.4236 42.7188) (width 0.25) (layer "B.Cu") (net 7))
 (segment (start 23.8215 41.1188) (end 23.8236 41.1188) (width 0.25) (layer "B.Cu") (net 7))
 (segment (start 25.1468 34.2188) (end 25.3215 34.2188) (width 0.25) (layer "F.Cu") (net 6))
 (segment (start 23.8215 34.2188) (end 25.1468 34.2188) (width 0.25) (layer "F.Cu") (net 6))
 (segment (start 28.75 41.9) (end 27.6247 41.9) (width 0.25) (layer "F.Cu") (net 6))
 (segment (start 25.3215 34.2188) (end 25.3215 39.5968) (width 0.25) (layer "F.Cu") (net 6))
 (segment (start 25.3215 39.5968) (end 27.6247 41.9) (width 0.25) (layer "F.Cu") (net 6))
 (segment (start 25.3215 34.2188) (end 25.4238 34.1165) (width 0.25) (layer "F.Cu") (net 6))
 (via (at 25.4238 34.1165) (size 0.8) (drill 0.4) (layers "F.Cu" "B.Cu") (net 6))
 (segment (start 23.8215 35.7188) (end 25.4238 34.1165) (width 0.25) (layer "B.Cu") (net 6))
 (segment (start 34.74 28.6753) (end 31.8 31.6153) (width 0.25) (layer "F.Cu") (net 26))
 (segment (start 34.74 27.5) (end 34.74 28.6753) (width 0.25) (layer "F.Cu") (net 26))
 (segment (start 31.8 31.6153) (end 31.8 35.65) (width 0.25) (layer "F.Cu") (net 26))
 (segment (start 34.74 27.5) (end 34.74 28.6753) (width 0.25) (layer "B.Cu") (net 26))
 (segment (start 30.9987 31.9024) (end 34.2258 28.6753) (width 0.25) (layer "B.Cu") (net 26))
 (segment (start 31.8 36.375) (end 30.9987 35.5737) (width 0.25) (layer "B.Cu") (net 26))
 (segment (start 34.2258 28.6753) (end 34.74 28.6753) (width 0.25) (layer "B.Cu") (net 26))
 (segment (start 30.9987 35.5737) (end 30.9987 31.9024) (width 0.25) (layer "B.Cu") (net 26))
 (segment (start 32.2 27.5) (end 32.2 28.6753) (width 0.25) (layer "F.Cu") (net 27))
 (segment (start 31 29.8753) (end 31 35.65) (width 0.25) (layer "F.Cu") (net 27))
 (segment (start 32.2 28.6753) (end 31 29.8753) (width 0.25) (layer "F.Cu") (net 27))
 (segment (start 38.3943 40.281) (end 38.3753 40.3) (width 0.25) (layer "F.Cu") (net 18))
 (segment (start 39.3124 40.281) (end 38.3943 40.281) (width 0.25) (layer "F.Cu") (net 18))
 (segment (start 37.25 40.3) (end 38.3753 40.3) (width 0.25) (layer "F.Cu") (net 18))
 (via (at 39.3124 40.281) (size 0.8) (drill 0.4) (layers "F.Cu" "B.Cu") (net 18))
 (segment (start 38.175 39.9) (end 38.9314 39.9) (width 0.25) (layer "B.Cu") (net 18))
 (segment (start 38.9314 39.9) (end 39.3124 40.281) (width 0.25) (layer "B.Cu") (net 18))
 (segment (start 40.0697 35.325) (end 39.2 35.325) (width 0.25) (layer "F.Cu") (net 2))
 (segment (start 37.4 33.5753) (end 33.5494 33.5753) (width 0.25) (layer "F.Cu") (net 2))
 (segment (start 32.6 35.65) (end 32.6 34.5247) (width 0.25) (layer "F.Cu") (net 2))
 (segment (start 39.2 35.325) (end 37.4503 33.5753) (width 0.25) (layer "F.Cu") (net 2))
 (segment (start 42 36.08) (end 40.8247 36.08) (width 0.25) (layer "F.Cu") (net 2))
 (segment (start 37.4 31.6) (end 37.4 32.6753) (width 0.25) (layer "F.Cu") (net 2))
 (segment (start 40.8247 36.08) (end 40.0697 35.325) (width 0.25) (layer "F.Cu") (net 2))
 (segment (start 37.4 33.5753) (end 37.4 32.6753) (width 0.25) (layer "F.Cu") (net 2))
 (segment (start 33.5494 33.5753) (end 32.6 34.5247) (width 0.25) (layer "F.Cu") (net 2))
 (segment (start 37.4503 33.5753) (end 37.4 33.5753) (width 0.25) (layer "F.Cu") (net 2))
 (segment (start 34.375 31.6) (end 38.855 36.08) (width 0.25) (layer "B.Cu") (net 2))
 (segment (start 38.855 36.08) (end 42 36.08) (width 0.25) (layer "B.Cu") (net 2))
 (segment (start 43.7 41.67) (end 42.8747 41.67) (width 0.25) (layer "F.Cu") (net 1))
 (segment (start 39.4865 37.075) (end 39.2 37.075) (width 0.25) (layer "F.Cu") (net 1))
 (segment (start 41.2 41.875) (end 38.4003 41.875) (width 0.25) (layer "F.Cu") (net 1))
 (segment (start 28.75 39.5) (end 27.6247 39.5) (width 0.25) (layer "F.Cu") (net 1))
 (segment (start 32.8067 41.1) (end 28.75 41.1) (width 0.25) (layer "F.Cu") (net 1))
 (segment (start 33.6067 41.9) (end 32.8067 41.1) (width 0.25) (layer "F.Cu") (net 1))
 (segment (start 42.5672 41.875) (end 42.7722 41.67) (width 0.25) (layer "F.Cu") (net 1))
 (segment (start 42.7722 40.3607) (end 39.4865 37.075) (width 0.25) (layer "F.Cu") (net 1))
 (segment (start 42.8747 41.67) (end 42.7722 41.67) (width 0.25) (layer "F.Cu") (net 1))
 (segment (start 38.4003 41.875) (end 38.3753 41.9) (width 0.25) (layer "F.Cu") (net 1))
 (segment (start 37.25 41.9) (end 33.6067 41.9) (width 0.25) (layer "F.Cu") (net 1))
 (segment (start 37.25 41.9) (end 38.3753 41.9) (width 0.25) (layer "F.Cu") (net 1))
 (segment (start 42.7722 41.67) (end 42.7722 40.3607) (width 0.25) (layer "F.Cu") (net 1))
 (segment (start 28.75 41.1) (end 27.6247 41.1) (width 0.25) (layer "F.Cu") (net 1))
 (segment (start 27.6247 41.1) (end 27.6247 39.5) (width 0.25) (layer "F.Cu") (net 1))
 (segment (start 41.2 41.875) (end 42.5672 41.875) (width 0.25) (layer "F.Cu") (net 1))
 (segment (start 44.54 31) (end 44.54 32.1753) (width 0.25) (layer "B.Cu") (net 1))
 (segment (start 46.2282 33.4962) (end 44.9073 32.1753) (width 0.25) (layer "B.Cu") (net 1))
 (segment (start 27.925 40.2438) (end 27.925 40.7) (width 0.25) (layer "B.Cu") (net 1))
 (segment (start 38.175 42.706) (end 38.175 42.8892) (width 0.25) (layer "B.Cu") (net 1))
 (segment (start 43.7 41.67) (end 44.5253 41.67) (width 0.25) (layer "B.Cu") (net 1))
 (segment (start 44.5253 41.67) (end 46.2282 39.9671) (width 0.25) (layer "B.Cu") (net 1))
 (segment (start 27.925 40.2438) (end 23.3481 40.2438) (width 0.25) (layer "B.Cu") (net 1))
 (segment (start 43.6742 41.67) (end 42.8747 41.67) (width 0.25) (layer "B.Cu") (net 1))
 (segment (start 27.925 40.7) (end 29.931 42.706) (width 0.25) (layer "B.Cu") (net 1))
 (segment (start 43.6742 41.67) (end 43.7 41.67) (width 0.25) (layer "B.Cu") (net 1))
 (segment (start 27.925 39.1) (end 27.925 40.2438) (width 0.25) (layer "B.Cu") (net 1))
 (segment (start 27.0798 30.625) (end 27.5 30.625) (width 0.25) (layer "B.Cu") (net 1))
 (segment (start 38.175 42.8892) (end 39.091 43.8052) (width 0.25) (layer "B.Cu") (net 1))
 (segment (start 22.9952 34.7096) (end 27.0798 30.625) (width 0.25) (layer "B.Cu") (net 1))
 (segment (start 23.3481 40.2438) (end 22.9952 39.8909) (width 0.25) (layer "B.Cu") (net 1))
 (segment (start 38.175 41.9) (end 38.175 42.706) (width 0.25) (layer "B.Cu") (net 1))
 (segment (start 22.9952 39.8909) (end 22.9952 34.7096) (width 0.25) (layer "B.Cu") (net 1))
 (segment (start 39.091 43.8052) (end 40.7395 43.8052) (width 0.25) (layer "B.Cu") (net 1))
 (segment (start 44.9073 32.1753) (end 44.54 32.1753) (width 0.25) (layer "B.Cu") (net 1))
 (segment (start 46.2282 39.9671) (end 46.2282 33.4962) (width 0.25) (layer "B.Cu") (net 1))
 (segment (start 29.931 42.706) (end 38.175 42.706) (width 0.25) (layer "B.Cu") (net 1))
 (segment (start 40.7395 43.8052) (end 42.8747 41.67) (width 0.25) (layer "B.Cu") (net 1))
 (segment (start 27.5 32.35) (end 27.475 32.375) (width 0.25) (layer "F.Cu") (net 29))
 (segment (start 27.475 32.375) (end 26.4153 32.375) (width 0.25) (layer "F.Cu") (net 29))
 (via (at 26.4153 32.375) (size 0.8) (drill 0.4) (layers "F.Cu" "B.Cu") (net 29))
 (segment (start 27.5 32.375) (end 26.4153 32.375) (width 0.25) (layer "B.Cu") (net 29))
 (segment (start 44.54 33.54) (end 46.2157 35.2157) (width 0.25) (layer "F.Cu") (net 14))
 (segment (start 46.2157 40.9637) (end 41.9041 45.2753) (width 0.25) (layer "F.Cu") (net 14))
 (segment (start 46.2157 35.2157) (end 46.2157 40.9637) (width 0.25) (layer "F.Cu") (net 14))
 (segment (start 35 44.15) (end 35 45.2753) (width 0.25) (layer "F.Cu") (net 14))
 (segment (start 41.9041 45.2753) (end 35 45.2753) (width 0.25) (layer "F.Cu") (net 14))
 (segment (start 39.451 43.0799) (end 38.3809 44.15) (width 0.25) (layer "F.Cu") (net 15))
 (segment (start 38.3809 44.15) (end 35.8 44.15) (width 0.25) (layer "F.Cu") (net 15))
 (via (at 39.451 43.0799) (size 0.8) (drill 0.4) (layers "F.Cu" "B.Cu") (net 15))
 (segment (start 44.109 34.81) (end 44.9355 34.81) (width 0.25) (layer "B.Cu") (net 15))
 (segment (start 44.9355 34.81) (end 45.7436 35.6181) (width 0.25) (layer "B.Cu") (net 15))
 (segment (start 42 32.1753) (end 42.3674 32.1753) (width 0.25) (layer "B.Cu") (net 15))
 (segment (start 45.7436 36.7873) (end 39.451 43.0799) (width 0.25) (layer "B.Cu") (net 15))
 (segment (start 42.3674 32.1753) (end 43.1753 32.9832) (width 0.25) (layer "B.Cu") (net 15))
 (segment (start 42 31) (end 42 32.1753) (width 0.25) (layer "B.Cu") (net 15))
 (segment (start 43.1753 32.9832) (end 43.1753 33.8763) (width 0.25) (layer "B.Cu") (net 15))
 (segment (start 45.7436 35.6181) (end 45.7436 36.7873) (width 0.25) (layer "B.Cu") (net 15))
 (segment (start 43.1753 33.8763) (end 44.109 34.81) (width 0.25) (layer "B.Cu") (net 15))
 (segment (start 43.7752 42.7641) (end 40.161 42.7641) (width 0.25) (layer "F.Cu") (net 16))
 (segment (start 42 33.54) (end 43.1753 33.54) (width 0.25) (layer "F.Cu") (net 16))
 (segment (start 43.1753 33.9074) (end 43.9832 34.7153) (width 0.25) (layer "F.Cu") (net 16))
 (segment (start 45.7653 40.774) (end 43.7752 42.7641) (width 0.25) (layer "F.Cu") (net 16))
 (segment (start 39.7515 42.3546) (end 38.7207 42.3546) (width 0.25) (layer "F.Cu") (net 16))
 (segment (start 40.161 42.7641) (end 39.7515 42.3546) (width 0.25) (layer "F.Cu") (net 16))
 (segment (start 37.25 42.7) (end 38.3753 42.7) (width 0.25) (layer "F.Cu") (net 16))
 (segment (start 38.7207 42.3546) (end 38.3753 42.7) (width 0.25) (layer "F.Cu") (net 16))
 (segment (start 43.9832 34.7153) (end 44.838 34.7153) (width 0.25) (layer "F.Cu") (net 16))
 (segment (start 43.1753 33.54) (end 43.1753 33.9074) (width 0.25) (layer "F.Cu") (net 16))
 (segment (start 44.838 34.7153) (end 45.7653 35.6426) (width 0.25) (layer "F.Cu") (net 16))
 (segment (start 45.7653 35.6426) (end 45.7653 40.774) (width 0.25) (layer "F.Cu") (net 16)))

